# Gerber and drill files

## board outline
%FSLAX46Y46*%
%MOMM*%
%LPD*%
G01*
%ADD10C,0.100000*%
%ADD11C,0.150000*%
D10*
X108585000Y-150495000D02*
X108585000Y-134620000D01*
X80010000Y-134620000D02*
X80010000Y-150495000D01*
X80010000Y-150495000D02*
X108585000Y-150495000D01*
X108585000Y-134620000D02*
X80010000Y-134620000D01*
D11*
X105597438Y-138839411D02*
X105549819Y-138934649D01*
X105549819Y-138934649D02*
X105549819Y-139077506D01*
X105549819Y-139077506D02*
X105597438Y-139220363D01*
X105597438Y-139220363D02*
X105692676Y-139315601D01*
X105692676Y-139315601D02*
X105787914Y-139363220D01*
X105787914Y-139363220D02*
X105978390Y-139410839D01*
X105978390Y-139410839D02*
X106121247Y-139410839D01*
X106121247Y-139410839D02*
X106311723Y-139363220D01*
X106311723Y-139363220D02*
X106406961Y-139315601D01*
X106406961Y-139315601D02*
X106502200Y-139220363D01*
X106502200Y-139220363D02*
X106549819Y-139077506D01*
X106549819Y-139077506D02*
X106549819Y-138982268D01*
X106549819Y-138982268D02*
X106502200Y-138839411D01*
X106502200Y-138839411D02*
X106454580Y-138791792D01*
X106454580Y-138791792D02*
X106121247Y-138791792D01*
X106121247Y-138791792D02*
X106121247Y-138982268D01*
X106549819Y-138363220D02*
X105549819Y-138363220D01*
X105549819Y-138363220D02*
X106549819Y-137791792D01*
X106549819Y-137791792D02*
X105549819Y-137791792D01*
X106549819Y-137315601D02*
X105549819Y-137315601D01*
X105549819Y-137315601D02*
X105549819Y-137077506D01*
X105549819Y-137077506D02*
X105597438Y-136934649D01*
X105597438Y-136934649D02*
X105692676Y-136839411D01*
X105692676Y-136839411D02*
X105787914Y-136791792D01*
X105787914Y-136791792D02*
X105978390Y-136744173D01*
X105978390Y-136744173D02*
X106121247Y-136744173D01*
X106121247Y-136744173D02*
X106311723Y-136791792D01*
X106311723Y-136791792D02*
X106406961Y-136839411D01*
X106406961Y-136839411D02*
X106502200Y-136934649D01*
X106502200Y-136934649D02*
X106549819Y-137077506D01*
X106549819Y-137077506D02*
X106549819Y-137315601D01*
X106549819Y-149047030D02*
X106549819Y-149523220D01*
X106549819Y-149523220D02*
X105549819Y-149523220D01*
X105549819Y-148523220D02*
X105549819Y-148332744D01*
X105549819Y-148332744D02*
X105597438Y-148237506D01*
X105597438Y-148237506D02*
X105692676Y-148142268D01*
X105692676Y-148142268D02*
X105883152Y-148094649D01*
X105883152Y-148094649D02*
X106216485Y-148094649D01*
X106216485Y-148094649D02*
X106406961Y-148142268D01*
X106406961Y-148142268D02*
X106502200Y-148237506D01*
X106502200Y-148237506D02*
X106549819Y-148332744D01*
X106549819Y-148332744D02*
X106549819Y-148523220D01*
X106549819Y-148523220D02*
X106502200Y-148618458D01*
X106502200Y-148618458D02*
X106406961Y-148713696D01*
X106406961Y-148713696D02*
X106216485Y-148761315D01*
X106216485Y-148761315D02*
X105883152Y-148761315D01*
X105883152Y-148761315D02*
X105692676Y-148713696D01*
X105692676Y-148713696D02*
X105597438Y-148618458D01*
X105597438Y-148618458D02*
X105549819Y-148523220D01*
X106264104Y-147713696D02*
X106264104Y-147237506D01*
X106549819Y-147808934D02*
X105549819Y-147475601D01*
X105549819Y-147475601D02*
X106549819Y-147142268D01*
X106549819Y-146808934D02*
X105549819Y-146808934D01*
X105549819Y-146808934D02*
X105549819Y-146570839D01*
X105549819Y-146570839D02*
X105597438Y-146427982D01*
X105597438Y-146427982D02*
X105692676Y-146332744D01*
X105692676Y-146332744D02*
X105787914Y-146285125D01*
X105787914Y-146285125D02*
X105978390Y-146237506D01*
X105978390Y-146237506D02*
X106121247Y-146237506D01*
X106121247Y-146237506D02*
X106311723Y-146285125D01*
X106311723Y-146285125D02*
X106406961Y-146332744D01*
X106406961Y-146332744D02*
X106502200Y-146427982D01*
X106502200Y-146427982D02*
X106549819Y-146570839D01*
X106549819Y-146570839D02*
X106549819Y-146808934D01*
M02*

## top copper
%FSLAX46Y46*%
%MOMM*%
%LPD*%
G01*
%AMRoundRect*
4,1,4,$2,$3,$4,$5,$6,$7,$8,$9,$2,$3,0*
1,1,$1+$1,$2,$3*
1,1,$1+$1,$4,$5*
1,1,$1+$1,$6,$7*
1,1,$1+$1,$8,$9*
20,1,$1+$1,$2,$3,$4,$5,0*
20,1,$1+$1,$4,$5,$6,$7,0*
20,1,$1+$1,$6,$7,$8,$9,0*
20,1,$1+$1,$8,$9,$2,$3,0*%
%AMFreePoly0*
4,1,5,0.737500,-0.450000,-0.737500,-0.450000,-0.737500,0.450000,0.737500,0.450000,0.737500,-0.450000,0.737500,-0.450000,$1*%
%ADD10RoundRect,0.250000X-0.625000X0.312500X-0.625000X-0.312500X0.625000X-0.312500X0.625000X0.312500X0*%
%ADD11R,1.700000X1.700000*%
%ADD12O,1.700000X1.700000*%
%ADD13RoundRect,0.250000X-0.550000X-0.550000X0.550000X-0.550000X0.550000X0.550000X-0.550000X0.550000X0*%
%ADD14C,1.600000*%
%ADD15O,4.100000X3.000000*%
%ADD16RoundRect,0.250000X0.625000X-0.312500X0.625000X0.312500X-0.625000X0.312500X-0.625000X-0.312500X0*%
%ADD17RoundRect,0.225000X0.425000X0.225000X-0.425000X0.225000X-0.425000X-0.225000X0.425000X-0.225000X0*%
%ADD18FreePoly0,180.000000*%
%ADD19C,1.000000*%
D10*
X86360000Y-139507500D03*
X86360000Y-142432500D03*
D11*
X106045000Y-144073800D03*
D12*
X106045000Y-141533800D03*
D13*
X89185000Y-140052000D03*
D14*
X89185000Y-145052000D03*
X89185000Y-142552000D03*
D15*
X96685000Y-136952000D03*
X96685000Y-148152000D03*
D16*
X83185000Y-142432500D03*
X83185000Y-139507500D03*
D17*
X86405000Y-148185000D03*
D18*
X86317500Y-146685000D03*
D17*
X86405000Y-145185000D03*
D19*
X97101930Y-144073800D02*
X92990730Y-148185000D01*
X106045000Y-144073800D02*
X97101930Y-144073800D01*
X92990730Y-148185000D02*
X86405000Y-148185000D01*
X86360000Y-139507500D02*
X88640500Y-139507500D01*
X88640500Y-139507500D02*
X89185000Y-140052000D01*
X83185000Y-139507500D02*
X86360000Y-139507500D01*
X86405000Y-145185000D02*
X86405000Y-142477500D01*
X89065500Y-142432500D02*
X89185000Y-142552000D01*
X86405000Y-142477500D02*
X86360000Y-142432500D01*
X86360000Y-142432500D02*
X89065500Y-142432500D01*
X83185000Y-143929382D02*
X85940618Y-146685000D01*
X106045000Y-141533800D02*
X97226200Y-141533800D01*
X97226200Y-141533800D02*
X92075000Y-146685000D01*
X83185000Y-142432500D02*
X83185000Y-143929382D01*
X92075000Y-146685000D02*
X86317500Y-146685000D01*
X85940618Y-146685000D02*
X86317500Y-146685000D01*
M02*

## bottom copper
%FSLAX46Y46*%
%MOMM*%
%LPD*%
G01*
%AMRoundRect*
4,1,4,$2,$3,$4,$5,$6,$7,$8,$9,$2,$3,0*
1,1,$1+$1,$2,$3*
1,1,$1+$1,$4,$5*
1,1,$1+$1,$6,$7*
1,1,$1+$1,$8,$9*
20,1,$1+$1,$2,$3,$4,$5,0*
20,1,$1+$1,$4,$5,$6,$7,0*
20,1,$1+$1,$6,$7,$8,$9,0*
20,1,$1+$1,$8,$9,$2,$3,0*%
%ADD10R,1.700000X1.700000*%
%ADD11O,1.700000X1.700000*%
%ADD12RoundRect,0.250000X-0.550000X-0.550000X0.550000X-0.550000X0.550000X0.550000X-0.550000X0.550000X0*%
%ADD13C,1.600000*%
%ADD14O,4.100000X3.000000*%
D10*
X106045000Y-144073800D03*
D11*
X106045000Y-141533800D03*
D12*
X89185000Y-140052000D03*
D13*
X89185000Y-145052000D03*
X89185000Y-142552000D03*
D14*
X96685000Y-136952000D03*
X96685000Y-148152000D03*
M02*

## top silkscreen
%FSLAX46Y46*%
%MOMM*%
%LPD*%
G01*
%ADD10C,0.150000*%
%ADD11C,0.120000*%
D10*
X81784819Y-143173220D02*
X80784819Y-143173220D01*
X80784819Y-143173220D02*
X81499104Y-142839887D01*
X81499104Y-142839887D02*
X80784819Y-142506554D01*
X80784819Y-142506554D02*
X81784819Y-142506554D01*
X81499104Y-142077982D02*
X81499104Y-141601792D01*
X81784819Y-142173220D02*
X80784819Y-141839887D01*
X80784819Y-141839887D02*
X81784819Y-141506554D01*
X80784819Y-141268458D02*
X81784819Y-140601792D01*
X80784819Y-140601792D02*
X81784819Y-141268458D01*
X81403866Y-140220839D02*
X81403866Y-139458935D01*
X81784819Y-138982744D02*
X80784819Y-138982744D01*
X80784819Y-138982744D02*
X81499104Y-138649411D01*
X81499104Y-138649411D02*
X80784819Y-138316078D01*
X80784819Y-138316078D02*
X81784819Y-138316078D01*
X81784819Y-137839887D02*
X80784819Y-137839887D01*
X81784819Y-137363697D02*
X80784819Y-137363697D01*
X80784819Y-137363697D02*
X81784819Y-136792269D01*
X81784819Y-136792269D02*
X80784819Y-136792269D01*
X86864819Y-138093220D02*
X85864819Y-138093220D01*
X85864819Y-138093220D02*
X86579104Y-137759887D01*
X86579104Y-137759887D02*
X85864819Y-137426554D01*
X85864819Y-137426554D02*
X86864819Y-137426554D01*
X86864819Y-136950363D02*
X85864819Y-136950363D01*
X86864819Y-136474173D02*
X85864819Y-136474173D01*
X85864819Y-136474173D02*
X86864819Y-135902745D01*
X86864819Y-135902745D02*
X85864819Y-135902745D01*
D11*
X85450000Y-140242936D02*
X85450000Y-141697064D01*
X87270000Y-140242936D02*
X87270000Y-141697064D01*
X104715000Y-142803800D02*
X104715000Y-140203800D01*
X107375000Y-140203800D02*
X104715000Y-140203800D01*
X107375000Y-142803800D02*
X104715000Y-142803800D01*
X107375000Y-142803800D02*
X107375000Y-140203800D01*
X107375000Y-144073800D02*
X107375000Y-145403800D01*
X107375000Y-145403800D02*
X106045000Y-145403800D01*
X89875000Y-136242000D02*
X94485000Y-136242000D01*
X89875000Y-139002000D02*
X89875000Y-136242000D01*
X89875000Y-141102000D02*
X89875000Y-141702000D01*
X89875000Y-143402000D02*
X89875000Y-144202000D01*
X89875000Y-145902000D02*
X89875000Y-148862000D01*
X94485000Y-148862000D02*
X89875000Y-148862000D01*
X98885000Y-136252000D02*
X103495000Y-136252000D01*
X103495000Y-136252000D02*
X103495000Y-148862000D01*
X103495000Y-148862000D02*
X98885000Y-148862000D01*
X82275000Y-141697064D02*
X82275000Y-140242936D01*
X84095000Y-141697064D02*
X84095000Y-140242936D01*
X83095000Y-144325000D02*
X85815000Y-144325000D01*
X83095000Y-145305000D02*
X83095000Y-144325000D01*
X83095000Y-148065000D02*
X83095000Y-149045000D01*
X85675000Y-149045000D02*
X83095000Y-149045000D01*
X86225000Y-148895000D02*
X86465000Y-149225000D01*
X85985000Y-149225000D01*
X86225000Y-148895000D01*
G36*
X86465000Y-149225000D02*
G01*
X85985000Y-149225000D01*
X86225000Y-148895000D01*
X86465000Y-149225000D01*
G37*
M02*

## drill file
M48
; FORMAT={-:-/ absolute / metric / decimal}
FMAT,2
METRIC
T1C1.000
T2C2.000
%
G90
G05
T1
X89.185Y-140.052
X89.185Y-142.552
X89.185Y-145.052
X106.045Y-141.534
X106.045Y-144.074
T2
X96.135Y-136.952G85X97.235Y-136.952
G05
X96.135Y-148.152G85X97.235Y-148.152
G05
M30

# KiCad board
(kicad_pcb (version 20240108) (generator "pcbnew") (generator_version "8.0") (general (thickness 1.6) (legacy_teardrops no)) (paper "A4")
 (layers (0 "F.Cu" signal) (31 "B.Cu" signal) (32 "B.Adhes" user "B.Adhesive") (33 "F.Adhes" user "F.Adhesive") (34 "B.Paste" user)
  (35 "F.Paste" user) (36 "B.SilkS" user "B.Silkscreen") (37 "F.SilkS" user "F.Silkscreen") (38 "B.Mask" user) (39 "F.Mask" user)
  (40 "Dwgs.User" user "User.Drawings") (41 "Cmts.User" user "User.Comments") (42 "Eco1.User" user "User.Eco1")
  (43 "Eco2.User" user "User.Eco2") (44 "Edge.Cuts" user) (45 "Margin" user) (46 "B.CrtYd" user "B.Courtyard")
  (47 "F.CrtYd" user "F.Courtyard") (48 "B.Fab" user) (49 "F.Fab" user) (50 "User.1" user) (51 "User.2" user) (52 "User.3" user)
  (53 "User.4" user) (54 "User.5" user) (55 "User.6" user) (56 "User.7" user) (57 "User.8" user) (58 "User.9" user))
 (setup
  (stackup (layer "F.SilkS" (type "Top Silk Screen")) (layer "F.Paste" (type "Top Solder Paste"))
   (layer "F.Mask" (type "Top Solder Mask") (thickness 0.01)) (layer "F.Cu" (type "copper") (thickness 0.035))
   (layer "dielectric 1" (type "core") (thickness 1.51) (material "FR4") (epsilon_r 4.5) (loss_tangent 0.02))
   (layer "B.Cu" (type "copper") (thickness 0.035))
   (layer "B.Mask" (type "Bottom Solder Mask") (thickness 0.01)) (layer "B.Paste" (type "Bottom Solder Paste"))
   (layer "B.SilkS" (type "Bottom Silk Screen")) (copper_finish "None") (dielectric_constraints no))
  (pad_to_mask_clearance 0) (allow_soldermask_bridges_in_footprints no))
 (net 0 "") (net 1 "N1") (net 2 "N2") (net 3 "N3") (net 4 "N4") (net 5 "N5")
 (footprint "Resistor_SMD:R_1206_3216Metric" (layer "F.Cu") (at 86.36 140.97 -90)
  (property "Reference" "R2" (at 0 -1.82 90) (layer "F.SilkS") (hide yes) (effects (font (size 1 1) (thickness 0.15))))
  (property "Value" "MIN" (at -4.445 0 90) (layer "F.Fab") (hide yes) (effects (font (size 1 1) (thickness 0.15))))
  (fp_line (start -0.727064 0.91) (end 0.727064 0.91) (stroke (width 0.12) (type solid)) (layer "F.SilkS"))
  (fp_line (start -0.727064 -0.91) (end 0.727064 -0.91) (stroke (width 0.12) (type solid)) (layer "F.SilkS"))
  (pad "1" smd roundrect (at -1.4625 0 270) (size 1.125 1.75) (layers "F.Cu" "F.Paste" "F.Mask") (roundrect_rratio 0.222222) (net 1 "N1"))
  (pad "2" smd roundrect (at 1.4625 0 270) (size 1.125 1.75) (layers "F.Cu" "F.Paste" "F.Mask") (roundrect_rratio 0.222222) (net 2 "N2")))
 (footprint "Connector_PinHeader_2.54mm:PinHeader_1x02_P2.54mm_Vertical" (layer "F.Cu") (at 106.045 144.0738 180)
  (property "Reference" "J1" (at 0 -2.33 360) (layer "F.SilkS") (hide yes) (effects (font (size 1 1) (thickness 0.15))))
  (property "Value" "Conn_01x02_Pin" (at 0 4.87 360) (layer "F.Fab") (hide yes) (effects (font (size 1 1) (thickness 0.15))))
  (fp_line (start 1.33 1.27) (end 1.33 3.87) (stroke (width 0.12) (type solid)) (layer "F.SilkS"))
  (fp_line (start -1.33 3.87) (end 1.33 3.87) (stroke (width 0.12) (type solid)) (layer "F.SilkS"))
  (fp_line (start -1.33 1.27) (end 1.33 1.27) (stroke (width 0.12) (type solid)) (layer "F.SilkS"))
  (fp_line (start -1.33 1.27) (end -1.33 3.87) (stroke (width 0.12) (type solid)) (layer "F.SilkS"))
  (fp_line (start -1.33 0) (end -1.33 -1.33) (stroke (width 0.12) (type solid)) (layer "F.SilkS"))
  (fp_line (start -1.33 -1.33) (end 0 -1.33) (stroke (width 0.12) (type solid)) (layer "F.SilkS"))
  (pad "1" thru_hole rect (at 0 0 180) (size 1.7 1.7) (drill 1) (layers "*.Cu" "*.Mask") (remove_unused_layers no) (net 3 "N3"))
  (pad "2" thru_hole oval (at 0 2.54 180) (size 1.7 1.7) (drill 1) (layers "*.Cu" "*.Mask") (remove_unused_layers no) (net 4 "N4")))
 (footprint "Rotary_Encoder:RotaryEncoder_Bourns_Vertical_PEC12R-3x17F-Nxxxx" (layer "F.Cu") (at 89.185 140.052)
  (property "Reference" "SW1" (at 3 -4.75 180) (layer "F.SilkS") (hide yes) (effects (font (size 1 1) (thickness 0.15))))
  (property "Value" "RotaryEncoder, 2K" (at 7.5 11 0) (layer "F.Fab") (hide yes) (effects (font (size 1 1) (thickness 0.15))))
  (fp_line (start 0.69 -3.81) (end 5.3 -3.81) (stroke (width 0.12) (type solid)) (layer "F.SilkS"))
  (fp_line (start 0.69 -1.05) (end 0.69 -3.81) (stroke (width 0.12) (type solid)) (layer "F.SilkS"))
  (fp_line (start 0.69 1.05) (end 0.69 1.65) (stroke (width 0.12) (type solid)) (layer "F.SilkS"))
  (fp_line (start 0.69 3.35) (end 0.69 4.15) (stroke (width 0.12) (type solid)) (layer "F.SilkS"))
  (fp_line (start 0.69 5.85) (end 0.69 8.81) (stroke (width 0.12) (type solid)) (layer "F.SilkS"))
  (fp_line (start 5.3 8.81) (end 0.69 8.81) (stroke (width 0.12) (type solid)) (layer "F.SilkS"))
  (fp_line (start 9.7 -3.8) (end 14.31 -3.8) (stroke (width 0.12) (type solid)) (layer "F.SilkS"))
  (fp_line (start 14.31 -3.8) (end 14.31 8.81) (stroke (width 0.12) (type solid)) (layer "F.SilkS"))
  (fp_line (start 14.31 8.81) (end 9.7 8.81) (stroke (width 0.12) (type solid)) (layer "F.SilkS"))
  (pad "A" thru_hole roundrect (at 0 0) (size 1.6 1.6) (drill 1) (layers "*.Cu" "*.Mask") (remove_unused_layers no)
   (roundrect_rratio 0.15625) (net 1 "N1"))
  (pad "B" thru_hole circle (at 0 5) (size 1.6 1.6) (drill 1) (layers "*.Cu" "*.Mask") (remove_unused_layers no) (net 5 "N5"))
  (pad "C" thru_hole circle (at 0 2.5) (size 1.6 1.6) (drill 1) (layers "*.Cu" "*.Mask") (remove_unused_layers no) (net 2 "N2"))
  (pad "SH" thru_hole oval (at 7.5 -3.1) (size 4.1 3) (drill oval 3.1 2) (layers "*.Cu" "*.Mask") (remove_unused_layers no))
  (pad "SH" thru_hole oval (at 7.5 8.1) (size 4.1 3) (drill oval 3.1 2) (layers "*.Cu" "*.Mask") (remove_unused_layers no)))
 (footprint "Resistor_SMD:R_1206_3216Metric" (layer "F.Cu") (at 83.185 140.97 90)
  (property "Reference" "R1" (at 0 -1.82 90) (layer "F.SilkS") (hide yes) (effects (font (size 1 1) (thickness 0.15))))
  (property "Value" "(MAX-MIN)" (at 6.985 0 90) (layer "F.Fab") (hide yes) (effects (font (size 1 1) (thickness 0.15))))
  (fp_line (start -0.727064 -0.91) (end 0.727064 -0.91) (stroke (width 0.12) (type solid)) (layer "F.SilkS"))
  (fp_line (start -0.727064 0.91) (end 0.727064 0.91) (stroke (width 0.12) (type solid)) (layer "F.SilkS"))
  (pad "1" smd roundrect (at -1.4625 0 90) (size 1.125 1.75) (layers "F.Cu" "F.Paste" "F.Mask") (roundrect_rratio 0.222222) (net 4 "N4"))
  (pad "2" smd roundrect (at 1.4625 0 90) (size 1.125 1.75) (layers "F.Cu" "F.Paste" "F.Mask") (roundrect_rratio 0.222222) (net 1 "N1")))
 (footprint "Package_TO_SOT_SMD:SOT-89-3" (layer "F.Cu") (at 84.455 146.685 180)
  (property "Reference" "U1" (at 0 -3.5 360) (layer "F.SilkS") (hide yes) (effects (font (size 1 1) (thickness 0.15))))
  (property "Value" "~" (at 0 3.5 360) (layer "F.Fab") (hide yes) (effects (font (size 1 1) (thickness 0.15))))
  (fp_line (start 1.36 2.36) (end -1.36 2.36) (stroke (width 0.12) (type solid)) (layer "F.SilkS"))
  (fp_line (start 1.36 1.38) (end 1.36 2.36) (stroke (width 0.12) (type solid)) (layer "F.SilkS"))
  (fp_line (start 1.36 -1.38) (end 1.36 -2.36) (stroke (width 0.12) (type solid)) (layer "F.SilkS"))
  (fp_line (start -1.22 -2.36) (end 1.36 -2.36) (stroke (width 0.12) (type solid)) (layer "F.SilkS"))
  (fp_poly
   (pts (xy -1.77 -2.21) (xy -2.01 -2.54) (xy -1.53 -2.54) (xy -1.77 -2.21)) (stroke (width 0.12) (type solid)) (fill solid)
   (layer "F.SilkS"))
  (pad "1" smd roundrect (at -1.95 -1.5 180) (size 1.3 0.9) (layers "F.Cu" "F.Paste" "F.Mask") (roundrect_rratio 0.25) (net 3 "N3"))
  (pad "2" smd custom (at -1.8625 0 180) (size 1.475 0.9) (layers "F.Cu" "F.Paste" "F.Mask") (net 4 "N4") (zone_connect 2)
   (thermal_bridge_angle 45) (options (clearance outline) (anchor rect)) (primitives))
  (pad "3" smd roundrect (at -1.95 1.5 180) (size 1.3 0.9) (layers "F.Cu" "F.Paste" "F.Mask") (roundrect_rratio 0.25) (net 2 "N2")))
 (gr_line (start 108.585 150.495) (end 108.585 134.62) (stroke (width 0.1) (type default)) (layer "Edge.Cuts"))
 (gr_line (start 80.01 134.62) (end 80.01 150.495) (stroke (width 0.1) (type default)) (layer "Edge.Cuts"))
 (gr_line (start 80.01 150.495) (end 108.585 150.495) (stroke (width 0.1) (type default)) (layer "Edge.Cuts"))
 (gr_line (start 108.585 134.62) (end 80.01 134.62) (stroke (width 0.1) (type default)) (layer "Edge.Cuts"))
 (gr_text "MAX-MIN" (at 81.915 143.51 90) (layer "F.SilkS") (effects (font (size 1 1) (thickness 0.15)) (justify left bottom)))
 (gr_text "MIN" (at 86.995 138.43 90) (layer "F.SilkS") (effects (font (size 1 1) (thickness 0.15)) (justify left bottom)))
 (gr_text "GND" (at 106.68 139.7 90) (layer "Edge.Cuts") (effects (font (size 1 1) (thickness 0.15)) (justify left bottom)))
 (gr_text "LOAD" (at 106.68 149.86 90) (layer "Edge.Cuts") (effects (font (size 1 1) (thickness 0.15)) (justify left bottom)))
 (segment (start 97.10193 144.0738) (end 92.99073 148.185) (width 1) (layer "F.Cu") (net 3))
 (segment (start 106.045 144.0738) (end 97.10193 144.0738) (width 1) (layer "F.Cu") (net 3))
 (segment (start 92.99073 148.185) (end 86.405 148.185) (width 1) (layer "F.Cu") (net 3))
 (segment (start 86.36 139.5075) (end 88.6405 139.5075) (width 1) (layer "F.Cu") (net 1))
 (segment (start 88.6405 139.5075) (end 89.185 140.052) (width 1) (layer "F.Cu") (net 1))
 (segment (start 83.185 139.5075) (end 86.36 139.5075) (width 1) (layer "F.Cu") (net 1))
 (segment (start 86.405 145.185) (end 86.405 142.4775) (width 1) (layer "F.Cu") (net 2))
 (segment (start 89.0655 142.4325) (end 89.185 142.552) (width 1) (layer "F.Cu") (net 2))
 (segment (start 86.405 142.4775) (end 86.36 142.4325) (width 1) (layer "F.Cu") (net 2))
 (segment (start 86.36 142.4325) (end 89.0655 142.4325) (width 1) (layer "F.Cu") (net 2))
 (segment (start 83.185 143.929382) (end 85.940618 146.685) (width 1) (layer "F.Cu") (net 4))
 (segment (start 106.045 141.5338) (end 97.2262 141.5338) (width 1) (layer "F.Cu") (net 4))
 (segment (start 97.2262 141.5338) (end 92.075 146.685) (width 1) (layer "F.Cu") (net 4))
 (segment (start 83.185 142.4325) (end 83.185 143.929382) (width 1) (layer "F.Cu") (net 4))
 (segment (start 92.075 146.685) (end 86.3175 146.685) (width 1) (layer "F.Cu") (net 4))
 (segment (start 85.940618 146.685) (end 86.3175 146.685) (width 1) (layer "F.Cu") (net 4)))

